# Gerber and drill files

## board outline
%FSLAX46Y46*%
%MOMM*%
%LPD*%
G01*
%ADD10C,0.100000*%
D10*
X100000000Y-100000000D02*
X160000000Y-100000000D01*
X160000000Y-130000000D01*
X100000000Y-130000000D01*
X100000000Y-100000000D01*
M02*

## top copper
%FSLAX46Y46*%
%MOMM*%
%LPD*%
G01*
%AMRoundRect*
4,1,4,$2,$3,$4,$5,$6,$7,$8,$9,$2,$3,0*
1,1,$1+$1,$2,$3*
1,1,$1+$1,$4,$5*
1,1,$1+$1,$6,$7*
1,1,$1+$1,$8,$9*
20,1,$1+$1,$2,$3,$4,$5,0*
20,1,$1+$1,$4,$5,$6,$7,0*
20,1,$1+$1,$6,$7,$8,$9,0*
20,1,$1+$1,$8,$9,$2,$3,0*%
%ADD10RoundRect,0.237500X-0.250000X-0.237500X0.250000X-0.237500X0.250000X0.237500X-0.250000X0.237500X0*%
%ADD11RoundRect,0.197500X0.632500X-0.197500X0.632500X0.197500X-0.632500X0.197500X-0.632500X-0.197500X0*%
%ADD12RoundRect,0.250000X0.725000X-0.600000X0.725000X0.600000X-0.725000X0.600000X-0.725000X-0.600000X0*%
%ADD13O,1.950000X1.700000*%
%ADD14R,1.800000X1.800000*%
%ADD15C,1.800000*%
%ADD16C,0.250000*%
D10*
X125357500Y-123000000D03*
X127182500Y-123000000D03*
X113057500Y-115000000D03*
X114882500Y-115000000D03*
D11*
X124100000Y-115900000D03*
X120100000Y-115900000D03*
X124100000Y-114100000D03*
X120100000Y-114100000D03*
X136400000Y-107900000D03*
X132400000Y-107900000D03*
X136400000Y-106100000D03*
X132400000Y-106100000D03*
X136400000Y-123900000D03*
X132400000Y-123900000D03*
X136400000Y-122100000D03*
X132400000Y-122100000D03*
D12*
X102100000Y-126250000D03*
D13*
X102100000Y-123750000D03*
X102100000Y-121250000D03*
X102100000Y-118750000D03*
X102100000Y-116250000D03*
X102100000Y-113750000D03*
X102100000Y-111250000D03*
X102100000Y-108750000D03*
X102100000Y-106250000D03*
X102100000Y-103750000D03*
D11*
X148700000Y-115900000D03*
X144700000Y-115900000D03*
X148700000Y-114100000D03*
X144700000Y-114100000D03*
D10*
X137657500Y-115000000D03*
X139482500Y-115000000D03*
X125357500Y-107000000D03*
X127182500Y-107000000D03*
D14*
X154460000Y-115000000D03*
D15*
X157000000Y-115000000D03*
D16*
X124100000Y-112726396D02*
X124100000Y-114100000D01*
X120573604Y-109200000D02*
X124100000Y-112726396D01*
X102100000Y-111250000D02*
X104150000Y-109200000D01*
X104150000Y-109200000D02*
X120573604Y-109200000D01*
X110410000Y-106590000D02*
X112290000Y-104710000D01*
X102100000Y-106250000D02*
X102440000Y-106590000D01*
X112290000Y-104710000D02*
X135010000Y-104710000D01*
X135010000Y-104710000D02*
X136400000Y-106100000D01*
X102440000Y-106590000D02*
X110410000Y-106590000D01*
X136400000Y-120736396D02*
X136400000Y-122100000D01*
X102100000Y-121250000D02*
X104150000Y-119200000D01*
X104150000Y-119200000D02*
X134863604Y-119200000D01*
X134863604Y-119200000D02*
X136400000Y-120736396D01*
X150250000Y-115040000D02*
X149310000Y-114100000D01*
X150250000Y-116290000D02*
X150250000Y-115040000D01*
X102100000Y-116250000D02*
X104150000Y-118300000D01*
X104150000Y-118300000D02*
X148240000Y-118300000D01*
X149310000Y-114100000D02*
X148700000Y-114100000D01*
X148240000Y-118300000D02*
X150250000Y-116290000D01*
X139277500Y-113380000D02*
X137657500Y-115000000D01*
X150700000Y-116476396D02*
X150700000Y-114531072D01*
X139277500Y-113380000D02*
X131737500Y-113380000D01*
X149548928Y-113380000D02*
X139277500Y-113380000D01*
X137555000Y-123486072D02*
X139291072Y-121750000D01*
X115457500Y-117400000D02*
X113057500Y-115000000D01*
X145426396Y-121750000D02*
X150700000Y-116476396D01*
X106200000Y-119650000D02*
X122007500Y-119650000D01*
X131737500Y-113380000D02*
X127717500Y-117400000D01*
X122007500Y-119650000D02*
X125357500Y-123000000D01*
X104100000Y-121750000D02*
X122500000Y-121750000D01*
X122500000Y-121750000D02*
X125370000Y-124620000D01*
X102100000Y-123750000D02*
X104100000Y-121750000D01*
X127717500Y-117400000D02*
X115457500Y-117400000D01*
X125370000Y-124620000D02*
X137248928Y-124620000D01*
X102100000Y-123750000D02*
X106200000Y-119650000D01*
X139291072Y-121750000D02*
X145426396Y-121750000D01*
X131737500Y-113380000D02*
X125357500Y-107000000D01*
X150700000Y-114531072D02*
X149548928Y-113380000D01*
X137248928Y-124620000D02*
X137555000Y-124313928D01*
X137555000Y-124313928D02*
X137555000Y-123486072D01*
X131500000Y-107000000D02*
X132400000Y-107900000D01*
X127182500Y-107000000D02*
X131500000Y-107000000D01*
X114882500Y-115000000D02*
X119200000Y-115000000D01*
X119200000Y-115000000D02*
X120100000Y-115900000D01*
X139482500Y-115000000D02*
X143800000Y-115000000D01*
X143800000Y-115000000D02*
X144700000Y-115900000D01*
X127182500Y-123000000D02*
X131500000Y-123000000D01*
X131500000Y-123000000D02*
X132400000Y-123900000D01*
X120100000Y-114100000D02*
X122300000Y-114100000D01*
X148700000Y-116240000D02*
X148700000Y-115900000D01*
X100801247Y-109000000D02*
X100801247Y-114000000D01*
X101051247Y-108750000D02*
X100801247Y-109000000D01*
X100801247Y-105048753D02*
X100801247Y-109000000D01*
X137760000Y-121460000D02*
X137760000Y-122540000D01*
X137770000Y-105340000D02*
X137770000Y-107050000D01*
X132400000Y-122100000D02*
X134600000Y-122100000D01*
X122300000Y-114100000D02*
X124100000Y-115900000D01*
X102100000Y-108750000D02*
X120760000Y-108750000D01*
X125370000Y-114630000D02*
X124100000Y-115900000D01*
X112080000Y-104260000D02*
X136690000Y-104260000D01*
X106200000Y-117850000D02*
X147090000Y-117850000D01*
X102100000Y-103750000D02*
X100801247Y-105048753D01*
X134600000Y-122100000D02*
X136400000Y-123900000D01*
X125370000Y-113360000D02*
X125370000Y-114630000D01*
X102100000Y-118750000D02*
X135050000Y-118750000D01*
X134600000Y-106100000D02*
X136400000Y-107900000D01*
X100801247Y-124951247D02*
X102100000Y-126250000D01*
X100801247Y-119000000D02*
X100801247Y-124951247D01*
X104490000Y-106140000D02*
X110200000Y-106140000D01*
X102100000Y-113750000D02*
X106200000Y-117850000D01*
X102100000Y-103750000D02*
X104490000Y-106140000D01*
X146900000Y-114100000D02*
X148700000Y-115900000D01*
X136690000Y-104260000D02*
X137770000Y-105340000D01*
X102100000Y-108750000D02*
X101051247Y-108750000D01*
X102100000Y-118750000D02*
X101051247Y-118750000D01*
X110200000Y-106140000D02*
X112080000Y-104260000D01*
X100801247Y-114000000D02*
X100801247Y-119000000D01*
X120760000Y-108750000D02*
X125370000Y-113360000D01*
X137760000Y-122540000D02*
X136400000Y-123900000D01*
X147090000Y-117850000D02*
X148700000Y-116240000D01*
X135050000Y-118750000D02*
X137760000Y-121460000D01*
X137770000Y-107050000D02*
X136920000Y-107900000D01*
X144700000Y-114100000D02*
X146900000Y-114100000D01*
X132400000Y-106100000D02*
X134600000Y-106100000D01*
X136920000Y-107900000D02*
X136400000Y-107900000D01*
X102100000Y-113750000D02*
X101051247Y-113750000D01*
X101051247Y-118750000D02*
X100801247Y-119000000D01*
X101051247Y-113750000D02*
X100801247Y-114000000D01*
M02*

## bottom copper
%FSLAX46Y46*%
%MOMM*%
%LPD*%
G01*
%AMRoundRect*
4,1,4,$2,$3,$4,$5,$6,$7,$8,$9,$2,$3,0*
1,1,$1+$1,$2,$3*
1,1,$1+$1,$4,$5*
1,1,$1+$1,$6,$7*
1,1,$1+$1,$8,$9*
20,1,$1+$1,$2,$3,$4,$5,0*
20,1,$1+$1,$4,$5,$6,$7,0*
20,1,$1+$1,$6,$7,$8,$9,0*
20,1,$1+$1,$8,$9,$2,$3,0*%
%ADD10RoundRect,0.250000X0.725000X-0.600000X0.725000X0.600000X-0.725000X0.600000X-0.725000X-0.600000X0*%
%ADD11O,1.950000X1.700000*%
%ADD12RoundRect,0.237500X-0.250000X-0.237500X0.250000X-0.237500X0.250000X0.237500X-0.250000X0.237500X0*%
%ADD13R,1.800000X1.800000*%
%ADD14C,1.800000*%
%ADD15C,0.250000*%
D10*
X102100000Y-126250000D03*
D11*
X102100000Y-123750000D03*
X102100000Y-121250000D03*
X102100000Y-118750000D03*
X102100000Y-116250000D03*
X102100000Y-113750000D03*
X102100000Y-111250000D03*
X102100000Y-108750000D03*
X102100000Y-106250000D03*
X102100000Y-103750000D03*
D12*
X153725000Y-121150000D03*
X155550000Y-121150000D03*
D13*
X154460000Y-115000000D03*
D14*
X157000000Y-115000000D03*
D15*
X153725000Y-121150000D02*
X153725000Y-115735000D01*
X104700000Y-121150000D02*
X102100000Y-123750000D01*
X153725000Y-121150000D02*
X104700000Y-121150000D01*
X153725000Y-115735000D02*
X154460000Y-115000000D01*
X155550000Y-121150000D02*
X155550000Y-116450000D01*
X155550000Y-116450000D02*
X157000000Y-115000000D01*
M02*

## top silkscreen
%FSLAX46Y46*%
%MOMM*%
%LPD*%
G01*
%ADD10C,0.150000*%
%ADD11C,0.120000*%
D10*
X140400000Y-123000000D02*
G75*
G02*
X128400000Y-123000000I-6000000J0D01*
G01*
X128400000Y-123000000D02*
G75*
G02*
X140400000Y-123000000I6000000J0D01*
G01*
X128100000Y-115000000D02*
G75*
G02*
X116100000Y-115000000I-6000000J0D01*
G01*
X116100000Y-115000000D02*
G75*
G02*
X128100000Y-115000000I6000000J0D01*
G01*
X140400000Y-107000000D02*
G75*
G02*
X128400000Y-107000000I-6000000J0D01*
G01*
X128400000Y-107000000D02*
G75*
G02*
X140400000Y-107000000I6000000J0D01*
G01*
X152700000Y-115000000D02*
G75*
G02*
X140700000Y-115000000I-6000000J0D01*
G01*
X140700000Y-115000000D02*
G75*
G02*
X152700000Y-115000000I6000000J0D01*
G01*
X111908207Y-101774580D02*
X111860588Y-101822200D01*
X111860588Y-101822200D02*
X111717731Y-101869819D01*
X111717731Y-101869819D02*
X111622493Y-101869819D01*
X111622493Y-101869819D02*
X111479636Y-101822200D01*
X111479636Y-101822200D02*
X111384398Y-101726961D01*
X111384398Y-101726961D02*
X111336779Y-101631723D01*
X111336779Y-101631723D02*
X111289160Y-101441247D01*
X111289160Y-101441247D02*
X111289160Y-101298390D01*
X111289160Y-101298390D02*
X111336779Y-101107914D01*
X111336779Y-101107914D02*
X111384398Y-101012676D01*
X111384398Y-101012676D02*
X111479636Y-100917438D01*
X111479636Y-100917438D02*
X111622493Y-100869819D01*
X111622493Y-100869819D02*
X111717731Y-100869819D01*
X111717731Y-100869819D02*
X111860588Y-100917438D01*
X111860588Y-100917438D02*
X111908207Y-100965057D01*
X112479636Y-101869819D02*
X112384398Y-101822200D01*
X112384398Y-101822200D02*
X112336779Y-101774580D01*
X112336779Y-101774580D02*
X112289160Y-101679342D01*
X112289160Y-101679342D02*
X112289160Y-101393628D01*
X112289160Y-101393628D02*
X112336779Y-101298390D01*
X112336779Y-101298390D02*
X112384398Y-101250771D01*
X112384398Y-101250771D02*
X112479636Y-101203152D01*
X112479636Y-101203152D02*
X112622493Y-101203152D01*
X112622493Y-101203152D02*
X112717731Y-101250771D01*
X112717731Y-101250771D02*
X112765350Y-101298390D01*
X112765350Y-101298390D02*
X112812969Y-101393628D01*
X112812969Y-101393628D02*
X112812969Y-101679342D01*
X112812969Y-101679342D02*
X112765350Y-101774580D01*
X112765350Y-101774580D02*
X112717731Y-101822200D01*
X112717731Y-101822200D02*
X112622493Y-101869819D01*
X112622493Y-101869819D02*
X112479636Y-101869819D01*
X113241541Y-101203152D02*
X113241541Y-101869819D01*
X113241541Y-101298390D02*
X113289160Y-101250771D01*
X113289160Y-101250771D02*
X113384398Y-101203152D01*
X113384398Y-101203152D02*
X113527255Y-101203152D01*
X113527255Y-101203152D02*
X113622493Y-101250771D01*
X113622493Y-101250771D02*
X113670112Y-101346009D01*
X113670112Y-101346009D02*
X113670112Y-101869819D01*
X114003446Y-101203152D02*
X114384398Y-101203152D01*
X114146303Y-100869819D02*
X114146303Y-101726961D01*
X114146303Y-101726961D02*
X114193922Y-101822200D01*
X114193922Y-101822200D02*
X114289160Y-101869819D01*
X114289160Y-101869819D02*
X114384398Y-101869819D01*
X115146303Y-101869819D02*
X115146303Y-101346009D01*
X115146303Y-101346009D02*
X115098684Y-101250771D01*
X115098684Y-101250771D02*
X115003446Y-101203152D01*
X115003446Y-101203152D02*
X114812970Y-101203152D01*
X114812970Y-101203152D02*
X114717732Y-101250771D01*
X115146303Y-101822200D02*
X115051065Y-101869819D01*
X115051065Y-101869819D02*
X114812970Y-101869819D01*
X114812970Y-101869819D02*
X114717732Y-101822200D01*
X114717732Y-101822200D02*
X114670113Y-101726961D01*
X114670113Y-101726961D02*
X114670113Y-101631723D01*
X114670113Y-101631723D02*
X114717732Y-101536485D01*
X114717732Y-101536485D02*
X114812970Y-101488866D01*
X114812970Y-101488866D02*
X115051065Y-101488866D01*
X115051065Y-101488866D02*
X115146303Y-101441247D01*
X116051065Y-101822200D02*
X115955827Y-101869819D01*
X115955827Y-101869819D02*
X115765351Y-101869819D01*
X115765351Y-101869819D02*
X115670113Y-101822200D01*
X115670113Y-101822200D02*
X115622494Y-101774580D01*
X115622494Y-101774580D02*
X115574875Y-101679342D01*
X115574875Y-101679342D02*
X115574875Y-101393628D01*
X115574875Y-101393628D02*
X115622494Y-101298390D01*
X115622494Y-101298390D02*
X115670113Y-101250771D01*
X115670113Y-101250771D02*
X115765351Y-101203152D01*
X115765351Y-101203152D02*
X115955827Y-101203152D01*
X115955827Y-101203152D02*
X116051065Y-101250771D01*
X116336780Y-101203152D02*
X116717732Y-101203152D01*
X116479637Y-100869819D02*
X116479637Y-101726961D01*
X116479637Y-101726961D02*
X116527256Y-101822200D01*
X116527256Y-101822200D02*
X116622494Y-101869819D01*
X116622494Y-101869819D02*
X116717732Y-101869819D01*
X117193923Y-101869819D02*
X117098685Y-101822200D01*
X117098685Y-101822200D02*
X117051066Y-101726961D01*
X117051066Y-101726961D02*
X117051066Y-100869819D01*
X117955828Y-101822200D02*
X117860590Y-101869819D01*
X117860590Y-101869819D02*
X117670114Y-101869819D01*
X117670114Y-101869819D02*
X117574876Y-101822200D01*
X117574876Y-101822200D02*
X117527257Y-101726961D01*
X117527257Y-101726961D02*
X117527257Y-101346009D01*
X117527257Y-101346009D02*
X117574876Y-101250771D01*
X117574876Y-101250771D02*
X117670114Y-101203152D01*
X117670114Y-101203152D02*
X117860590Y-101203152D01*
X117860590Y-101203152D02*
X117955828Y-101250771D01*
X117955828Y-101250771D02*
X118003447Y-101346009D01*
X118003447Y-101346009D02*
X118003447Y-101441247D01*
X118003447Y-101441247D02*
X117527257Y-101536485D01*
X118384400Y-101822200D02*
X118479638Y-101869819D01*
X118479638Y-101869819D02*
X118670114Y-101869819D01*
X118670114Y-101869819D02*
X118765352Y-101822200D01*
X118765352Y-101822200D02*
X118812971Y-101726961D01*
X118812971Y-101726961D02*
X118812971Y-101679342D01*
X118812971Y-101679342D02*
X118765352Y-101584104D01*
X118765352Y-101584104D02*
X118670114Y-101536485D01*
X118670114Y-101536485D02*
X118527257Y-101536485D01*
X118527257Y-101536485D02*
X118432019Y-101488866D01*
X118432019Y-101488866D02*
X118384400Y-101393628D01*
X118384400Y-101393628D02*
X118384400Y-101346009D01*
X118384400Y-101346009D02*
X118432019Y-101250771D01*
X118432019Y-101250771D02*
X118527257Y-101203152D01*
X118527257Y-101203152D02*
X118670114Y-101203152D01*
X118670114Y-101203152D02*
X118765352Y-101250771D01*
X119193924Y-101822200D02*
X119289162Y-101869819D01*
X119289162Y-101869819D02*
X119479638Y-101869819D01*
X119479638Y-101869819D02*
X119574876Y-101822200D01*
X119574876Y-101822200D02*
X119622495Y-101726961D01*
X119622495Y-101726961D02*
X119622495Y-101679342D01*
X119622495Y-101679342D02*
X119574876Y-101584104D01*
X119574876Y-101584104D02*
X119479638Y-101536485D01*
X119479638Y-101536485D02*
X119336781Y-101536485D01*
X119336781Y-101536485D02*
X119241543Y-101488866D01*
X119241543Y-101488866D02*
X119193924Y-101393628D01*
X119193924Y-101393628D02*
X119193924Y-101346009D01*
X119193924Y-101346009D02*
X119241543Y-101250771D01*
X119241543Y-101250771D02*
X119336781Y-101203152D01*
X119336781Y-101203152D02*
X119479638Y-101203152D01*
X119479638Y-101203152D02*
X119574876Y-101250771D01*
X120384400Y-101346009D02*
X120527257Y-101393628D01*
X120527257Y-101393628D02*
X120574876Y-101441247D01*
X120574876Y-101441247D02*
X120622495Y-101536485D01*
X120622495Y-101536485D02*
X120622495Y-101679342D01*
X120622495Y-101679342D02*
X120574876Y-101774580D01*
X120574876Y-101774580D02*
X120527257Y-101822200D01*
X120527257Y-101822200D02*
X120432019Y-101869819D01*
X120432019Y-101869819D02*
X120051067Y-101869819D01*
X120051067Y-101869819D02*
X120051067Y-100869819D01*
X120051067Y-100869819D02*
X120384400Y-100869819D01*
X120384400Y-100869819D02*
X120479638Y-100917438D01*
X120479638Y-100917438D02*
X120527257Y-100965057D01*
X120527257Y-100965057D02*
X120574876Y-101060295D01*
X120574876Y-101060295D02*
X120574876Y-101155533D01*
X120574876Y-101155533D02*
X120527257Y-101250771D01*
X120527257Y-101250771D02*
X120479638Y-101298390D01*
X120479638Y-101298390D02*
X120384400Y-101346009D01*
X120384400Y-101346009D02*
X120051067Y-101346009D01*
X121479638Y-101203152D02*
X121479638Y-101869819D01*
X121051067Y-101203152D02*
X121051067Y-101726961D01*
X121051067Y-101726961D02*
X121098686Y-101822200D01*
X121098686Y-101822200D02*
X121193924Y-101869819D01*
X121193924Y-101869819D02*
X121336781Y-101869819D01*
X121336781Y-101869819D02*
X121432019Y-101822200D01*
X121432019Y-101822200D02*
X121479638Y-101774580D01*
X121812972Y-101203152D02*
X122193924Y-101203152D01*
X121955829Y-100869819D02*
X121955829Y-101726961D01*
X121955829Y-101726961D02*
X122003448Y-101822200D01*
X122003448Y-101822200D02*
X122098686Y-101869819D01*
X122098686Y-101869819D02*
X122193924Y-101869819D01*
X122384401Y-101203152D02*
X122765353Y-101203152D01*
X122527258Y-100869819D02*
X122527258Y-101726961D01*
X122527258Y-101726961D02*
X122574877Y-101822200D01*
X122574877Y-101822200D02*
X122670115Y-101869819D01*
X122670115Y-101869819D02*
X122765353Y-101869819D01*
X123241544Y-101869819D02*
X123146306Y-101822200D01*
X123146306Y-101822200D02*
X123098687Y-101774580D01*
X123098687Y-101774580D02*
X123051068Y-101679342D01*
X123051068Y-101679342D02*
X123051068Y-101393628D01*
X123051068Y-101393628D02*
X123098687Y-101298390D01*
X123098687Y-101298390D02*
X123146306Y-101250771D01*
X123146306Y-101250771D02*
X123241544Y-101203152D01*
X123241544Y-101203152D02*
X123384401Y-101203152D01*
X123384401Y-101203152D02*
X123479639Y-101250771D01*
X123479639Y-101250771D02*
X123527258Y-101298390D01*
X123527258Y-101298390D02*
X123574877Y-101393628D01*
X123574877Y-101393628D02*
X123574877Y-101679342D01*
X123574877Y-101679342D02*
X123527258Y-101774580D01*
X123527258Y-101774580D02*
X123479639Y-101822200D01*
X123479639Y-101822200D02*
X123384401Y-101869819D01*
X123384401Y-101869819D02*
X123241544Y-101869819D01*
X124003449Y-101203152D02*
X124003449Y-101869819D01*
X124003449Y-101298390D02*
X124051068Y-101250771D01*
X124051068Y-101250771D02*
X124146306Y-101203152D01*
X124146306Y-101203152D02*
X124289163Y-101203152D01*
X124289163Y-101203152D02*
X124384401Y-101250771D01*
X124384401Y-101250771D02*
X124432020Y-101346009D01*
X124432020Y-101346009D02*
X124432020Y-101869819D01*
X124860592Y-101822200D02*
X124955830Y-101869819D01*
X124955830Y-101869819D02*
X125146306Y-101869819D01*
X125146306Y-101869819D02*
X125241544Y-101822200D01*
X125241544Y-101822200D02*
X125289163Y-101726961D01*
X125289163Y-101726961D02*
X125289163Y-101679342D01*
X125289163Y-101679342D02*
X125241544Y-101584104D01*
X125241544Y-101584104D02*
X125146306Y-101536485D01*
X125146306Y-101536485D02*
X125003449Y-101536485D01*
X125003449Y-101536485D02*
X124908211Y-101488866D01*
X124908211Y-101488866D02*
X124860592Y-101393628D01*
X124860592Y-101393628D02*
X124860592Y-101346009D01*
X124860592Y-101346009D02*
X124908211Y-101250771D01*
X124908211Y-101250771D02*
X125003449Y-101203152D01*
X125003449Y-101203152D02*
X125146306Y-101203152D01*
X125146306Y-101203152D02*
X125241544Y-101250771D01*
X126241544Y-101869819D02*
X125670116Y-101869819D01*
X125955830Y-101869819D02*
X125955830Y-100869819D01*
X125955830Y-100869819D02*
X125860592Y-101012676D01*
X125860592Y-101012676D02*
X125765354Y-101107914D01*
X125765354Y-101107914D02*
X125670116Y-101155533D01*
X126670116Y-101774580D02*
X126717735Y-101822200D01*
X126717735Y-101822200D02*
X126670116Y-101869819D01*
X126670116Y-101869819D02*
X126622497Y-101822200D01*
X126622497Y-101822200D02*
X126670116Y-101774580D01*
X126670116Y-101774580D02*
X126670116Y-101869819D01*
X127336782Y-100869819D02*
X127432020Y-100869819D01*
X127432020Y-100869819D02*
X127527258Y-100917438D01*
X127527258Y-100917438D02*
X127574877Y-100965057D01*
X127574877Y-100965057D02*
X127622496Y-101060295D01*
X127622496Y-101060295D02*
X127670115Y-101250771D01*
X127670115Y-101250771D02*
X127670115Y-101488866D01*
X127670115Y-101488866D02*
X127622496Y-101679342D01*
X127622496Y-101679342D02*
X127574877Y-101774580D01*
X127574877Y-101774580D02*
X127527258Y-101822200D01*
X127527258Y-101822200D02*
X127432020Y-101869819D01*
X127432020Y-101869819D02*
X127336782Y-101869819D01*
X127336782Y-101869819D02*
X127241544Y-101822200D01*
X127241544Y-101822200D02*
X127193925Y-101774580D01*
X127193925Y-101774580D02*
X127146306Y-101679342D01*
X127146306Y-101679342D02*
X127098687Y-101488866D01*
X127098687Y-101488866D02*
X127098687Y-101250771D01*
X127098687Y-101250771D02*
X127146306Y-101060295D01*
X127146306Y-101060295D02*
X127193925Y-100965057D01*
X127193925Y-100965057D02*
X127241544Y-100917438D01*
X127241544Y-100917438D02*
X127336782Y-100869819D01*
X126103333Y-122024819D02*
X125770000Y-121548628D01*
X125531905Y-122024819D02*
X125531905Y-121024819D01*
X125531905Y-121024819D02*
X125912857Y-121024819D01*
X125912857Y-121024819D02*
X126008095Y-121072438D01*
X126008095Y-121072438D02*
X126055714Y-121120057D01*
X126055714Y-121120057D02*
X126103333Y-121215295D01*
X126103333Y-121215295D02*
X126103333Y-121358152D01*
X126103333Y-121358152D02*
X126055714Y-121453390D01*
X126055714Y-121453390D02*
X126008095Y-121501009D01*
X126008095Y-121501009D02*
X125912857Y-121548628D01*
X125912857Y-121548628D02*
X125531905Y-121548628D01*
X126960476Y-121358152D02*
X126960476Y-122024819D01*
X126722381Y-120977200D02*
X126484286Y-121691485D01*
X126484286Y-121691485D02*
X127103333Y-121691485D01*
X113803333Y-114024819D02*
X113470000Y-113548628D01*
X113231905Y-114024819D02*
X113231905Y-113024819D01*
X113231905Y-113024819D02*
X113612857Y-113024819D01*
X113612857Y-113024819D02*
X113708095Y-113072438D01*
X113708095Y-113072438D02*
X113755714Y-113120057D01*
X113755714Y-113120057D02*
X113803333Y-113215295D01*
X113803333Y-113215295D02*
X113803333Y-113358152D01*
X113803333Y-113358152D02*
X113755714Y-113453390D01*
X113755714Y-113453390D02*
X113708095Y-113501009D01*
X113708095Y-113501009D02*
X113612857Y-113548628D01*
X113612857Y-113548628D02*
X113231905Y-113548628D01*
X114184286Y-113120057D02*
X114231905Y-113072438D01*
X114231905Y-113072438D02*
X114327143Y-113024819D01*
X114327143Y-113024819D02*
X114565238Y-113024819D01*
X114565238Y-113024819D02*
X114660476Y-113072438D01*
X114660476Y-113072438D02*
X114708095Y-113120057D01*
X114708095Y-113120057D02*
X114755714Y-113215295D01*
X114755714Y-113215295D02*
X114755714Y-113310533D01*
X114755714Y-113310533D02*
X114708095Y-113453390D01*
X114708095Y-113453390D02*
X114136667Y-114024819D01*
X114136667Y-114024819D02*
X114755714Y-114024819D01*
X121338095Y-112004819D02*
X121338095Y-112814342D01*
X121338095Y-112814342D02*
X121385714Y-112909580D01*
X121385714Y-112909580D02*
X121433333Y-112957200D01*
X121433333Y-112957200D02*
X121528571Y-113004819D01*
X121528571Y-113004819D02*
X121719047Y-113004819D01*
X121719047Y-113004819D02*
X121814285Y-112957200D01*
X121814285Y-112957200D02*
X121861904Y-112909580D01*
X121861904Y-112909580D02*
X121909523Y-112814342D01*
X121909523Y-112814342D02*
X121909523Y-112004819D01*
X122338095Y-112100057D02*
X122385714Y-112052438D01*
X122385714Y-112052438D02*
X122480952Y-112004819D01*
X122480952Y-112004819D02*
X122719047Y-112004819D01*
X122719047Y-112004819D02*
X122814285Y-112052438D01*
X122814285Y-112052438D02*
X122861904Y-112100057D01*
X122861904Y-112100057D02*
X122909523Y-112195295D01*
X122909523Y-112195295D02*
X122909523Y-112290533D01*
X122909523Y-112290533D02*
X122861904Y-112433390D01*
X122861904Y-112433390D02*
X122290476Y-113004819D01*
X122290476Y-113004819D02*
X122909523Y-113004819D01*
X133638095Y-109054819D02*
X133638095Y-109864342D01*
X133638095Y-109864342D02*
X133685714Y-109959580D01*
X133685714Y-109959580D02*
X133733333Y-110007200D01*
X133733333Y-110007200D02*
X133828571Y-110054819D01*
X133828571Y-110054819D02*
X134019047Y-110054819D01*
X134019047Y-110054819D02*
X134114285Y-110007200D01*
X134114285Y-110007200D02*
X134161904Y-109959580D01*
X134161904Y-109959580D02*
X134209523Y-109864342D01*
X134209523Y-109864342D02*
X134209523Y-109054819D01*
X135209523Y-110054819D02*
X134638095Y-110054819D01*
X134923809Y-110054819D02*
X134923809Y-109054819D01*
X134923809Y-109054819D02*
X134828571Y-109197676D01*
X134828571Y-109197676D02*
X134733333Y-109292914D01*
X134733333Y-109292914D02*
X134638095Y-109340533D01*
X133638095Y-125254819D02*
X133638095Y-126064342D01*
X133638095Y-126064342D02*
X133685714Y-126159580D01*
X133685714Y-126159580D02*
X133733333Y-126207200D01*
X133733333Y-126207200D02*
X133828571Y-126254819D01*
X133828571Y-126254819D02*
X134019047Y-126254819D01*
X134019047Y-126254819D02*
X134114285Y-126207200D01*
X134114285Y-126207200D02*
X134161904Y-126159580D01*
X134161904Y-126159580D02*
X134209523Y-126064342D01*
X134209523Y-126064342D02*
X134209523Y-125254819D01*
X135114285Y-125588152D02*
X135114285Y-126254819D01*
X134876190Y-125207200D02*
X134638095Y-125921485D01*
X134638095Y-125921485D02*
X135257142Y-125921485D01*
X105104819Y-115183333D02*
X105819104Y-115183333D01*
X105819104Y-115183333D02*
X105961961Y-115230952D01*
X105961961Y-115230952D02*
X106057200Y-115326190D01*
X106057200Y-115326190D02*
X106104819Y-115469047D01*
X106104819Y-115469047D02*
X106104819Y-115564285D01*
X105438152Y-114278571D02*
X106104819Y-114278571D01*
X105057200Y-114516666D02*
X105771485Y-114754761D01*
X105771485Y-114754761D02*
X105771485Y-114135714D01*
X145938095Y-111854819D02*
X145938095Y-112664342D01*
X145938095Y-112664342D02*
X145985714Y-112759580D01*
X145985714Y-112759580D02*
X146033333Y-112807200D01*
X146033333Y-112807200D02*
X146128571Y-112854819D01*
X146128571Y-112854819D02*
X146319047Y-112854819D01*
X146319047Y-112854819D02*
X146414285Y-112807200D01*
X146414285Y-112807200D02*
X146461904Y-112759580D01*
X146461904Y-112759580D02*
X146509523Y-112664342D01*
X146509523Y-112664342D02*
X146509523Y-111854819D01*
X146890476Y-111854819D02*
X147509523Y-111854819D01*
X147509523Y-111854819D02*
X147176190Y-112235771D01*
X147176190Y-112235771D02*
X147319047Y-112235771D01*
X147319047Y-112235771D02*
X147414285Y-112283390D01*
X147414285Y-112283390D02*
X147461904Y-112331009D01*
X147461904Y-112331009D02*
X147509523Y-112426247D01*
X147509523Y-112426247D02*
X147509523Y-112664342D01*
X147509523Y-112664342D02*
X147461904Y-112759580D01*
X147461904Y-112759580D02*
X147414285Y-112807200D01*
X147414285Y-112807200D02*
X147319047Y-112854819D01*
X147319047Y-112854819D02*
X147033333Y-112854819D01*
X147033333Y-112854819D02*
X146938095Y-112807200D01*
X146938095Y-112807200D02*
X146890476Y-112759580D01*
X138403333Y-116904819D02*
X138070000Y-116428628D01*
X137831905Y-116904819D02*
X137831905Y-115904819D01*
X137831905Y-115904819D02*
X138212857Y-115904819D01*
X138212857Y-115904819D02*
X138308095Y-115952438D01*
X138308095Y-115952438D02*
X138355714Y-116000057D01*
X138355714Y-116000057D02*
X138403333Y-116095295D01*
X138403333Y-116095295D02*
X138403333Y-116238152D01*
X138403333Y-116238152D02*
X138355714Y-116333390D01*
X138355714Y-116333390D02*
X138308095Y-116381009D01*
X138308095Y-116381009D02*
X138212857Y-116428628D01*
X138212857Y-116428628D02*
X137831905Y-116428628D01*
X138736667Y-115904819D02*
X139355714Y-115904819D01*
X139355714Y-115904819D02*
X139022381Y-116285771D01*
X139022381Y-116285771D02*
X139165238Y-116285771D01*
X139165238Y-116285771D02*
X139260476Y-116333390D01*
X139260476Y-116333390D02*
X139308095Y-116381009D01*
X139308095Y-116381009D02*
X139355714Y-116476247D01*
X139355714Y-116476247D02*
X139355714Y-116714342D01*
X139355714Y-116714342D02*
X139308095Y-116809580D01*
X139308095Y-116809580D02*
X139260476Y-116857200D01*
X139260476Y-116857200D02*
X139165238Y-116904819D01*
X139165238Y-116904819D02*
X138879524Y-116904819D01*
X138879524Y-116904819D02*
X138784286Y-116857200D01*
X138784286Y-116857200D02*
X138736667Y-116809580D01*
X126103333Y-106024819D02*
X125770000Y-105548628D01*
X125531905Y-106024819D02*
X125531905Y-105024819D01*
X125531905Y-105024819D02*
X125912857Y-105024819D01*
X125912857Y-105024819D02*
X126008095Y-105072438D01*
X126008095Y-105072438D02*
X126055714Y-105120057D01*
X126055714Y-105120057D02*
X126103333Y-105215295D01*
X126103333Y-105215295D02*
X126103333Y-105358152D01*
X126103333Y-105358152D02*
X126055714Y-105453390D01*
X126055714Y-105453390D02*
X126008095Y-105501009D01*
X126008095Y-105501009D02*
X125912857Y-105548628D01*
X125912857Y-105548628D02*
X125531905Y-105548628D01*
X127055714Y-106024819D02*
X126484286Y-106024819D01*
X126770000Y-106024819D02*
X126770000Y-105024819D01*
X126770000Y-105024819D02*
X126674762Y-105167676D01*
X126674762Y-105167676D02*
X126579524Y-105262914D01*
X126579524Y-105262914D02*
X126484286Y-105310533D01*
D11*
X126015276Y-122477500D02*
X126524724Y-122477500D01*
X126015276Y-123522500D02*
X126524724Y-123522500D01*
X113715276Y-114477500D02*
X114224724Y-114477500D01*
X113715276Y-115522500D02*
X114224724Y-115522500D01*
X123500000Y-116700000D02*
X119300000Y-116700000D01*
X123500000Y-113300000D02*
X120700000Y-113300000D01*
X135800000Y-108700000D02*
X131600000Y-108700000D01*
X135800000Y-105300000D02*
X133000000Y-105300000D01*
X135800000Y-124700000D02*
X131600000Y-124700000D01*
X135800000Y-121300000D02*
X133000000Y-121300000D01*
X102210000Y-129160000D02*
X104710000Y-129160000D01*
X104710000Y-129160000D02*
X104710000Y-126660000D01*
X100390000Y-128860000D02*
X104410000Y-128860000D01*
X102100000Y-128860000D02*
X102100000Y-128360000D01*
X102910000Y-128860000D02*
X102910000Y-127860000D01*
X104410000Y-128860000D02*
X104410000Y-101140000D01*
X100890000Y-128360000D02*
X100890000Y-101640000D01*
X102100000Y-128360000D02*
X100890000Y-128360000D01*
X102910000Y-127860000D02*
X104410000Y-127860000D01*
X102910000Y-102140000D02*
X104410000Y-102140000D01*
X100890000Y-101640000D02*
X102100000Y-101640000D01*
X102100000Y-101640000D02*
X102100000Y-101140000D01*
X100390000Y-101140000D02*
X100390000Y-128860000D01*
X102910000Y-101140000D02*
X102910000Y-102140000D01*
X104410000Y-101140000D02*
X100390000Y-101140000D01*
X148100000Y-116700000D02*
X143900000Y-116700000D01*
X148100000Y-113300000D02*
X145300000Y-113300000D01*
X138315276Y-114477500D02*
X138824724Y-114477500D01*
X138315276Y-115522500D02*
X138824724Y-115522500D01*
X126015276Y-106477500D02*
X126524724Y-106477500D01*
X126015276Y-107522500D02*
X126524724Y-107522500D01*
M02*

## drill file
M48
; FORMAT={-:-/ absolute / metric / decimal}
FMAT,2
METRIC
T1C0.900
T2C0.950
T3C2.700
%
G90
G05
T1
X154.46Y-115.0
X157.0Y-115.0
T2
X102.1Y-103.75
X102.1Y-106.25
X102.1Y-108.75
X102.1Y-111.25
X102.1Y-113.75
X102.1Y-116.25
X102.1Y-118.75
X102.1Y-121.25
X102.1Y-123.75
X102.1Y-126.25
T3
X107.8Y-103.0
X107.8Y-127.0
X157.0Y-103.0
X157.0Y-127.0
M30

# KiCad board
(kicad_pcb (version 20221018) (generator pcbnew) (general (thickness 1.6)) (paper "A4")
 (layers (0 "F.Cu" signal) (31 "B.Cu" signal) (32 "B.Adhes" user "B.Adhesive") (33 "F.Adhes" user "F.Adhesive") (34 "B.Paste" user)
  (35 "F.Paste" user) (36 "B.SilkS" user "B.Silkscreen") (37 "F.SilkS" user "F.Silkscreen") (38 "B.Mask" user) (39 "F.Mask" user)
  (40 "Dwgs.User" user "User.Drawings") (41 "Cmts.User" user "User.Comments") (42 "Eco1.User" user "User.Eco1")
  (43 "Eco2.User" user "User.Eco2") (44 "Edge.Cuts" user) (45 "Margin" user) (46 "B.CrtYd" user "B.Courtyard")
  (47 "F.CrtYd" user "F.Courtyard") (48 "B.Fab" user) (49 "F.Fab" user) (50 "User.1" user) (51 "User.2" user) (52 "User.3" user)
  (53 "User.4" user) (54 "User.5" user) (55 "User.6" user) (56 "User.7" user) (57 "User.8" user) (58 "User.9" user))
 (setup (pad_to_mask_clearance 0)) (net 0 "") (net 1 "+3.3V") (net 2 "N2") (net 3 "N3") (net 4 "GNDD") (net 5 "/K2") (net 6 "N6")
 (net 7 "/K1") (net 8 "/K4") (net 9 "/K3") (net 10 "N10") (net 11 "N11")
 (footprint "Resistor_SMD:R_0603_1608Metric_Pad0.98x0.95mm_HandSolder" (layer "F.Cu") (at 126.27 123)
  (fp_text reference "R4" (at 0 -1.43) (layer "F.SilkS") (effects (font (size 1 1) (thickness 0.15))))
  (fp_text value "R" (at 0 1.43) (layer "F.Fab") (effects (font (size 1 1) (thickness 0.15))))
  (fp_line (start -0.254724 -0.5225) (end 0.254724 -0.5225) (stroke (width 0.12) (type solid)) (layer "F.SilkS"))
  (fp_line (start -0.254724 0.5225) (end 0.254724 0.5225) (stroke (width 0.12) (type solid)) (layer "F.SilkS"))
  (pad "1" smd roundrect (at -0.9125 0) (size 0.975 0.95) (layers "F.Cu" "F.Paste" "F.Mask") (roundrect_rratio 0.25) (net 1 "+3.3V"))
  (pad "2" smd roundrect (at 0.9125 0) (size 0.975 0.95) (layers "F.Cu" "F.Paste" "F.Mask") (roundrect_rratio 0.25) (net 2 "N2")))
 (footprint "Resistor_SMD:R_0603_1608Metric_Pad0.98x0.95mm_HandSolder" (layer "F.Cu") (at 113.97 115)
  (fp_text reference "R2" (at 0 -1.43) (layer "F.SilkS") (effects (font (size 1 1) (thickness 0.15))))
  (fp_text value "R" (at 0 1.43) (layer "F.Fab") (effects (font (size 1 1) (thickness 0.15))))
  (fp_line (start -0.254724 -0.5225) (end 0.254724 -0.5225) (stroke (width 0.12) (type solid)) (layer "F.SilkS"))
  (fp_line (start -0.254724 0.5225) (end 0.254724 0.5225) (stroke (width 0.12) (type solid)) (layer "F.SilkS"))
  (pad "1" smd roundrect (at -0.9125 0) (size 0.975 0.95) (layers "F.Cu" "F.Paste" "F.Mask") (roundrect_rratio 0.25) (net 1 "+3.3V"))
  (pad "2" smd roundrect (at 0.9125 0) (size 0.975 0.95) (layers "F.Cu" "F.Paste" "F.Mask") (roundrect_rratio 0.25) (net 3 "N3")))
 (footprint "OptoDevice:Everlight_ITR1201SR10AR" (layer "F.Cu") (at 122.1 115 90)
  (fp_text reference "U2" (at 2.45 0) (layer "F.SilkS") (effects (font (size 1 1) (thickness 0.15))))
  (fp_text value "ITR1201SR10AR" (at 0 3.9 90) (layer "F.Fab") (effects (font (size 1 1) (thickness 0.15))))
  (fp_line (start -1.7 1.4) (end -1.7 -2.8) (stroke (width 0.12) (type solid)) (layer "F.SilkS"))
  (fp_line (start 1.7 1.4) (end 1.7 -1.4) (stroke (width 0.12) (type solid)) (layer "F.SilkS"))
  (pad "1" smd roundrect (at -0.9 2 90) (size 0.79 1.66) (layers "F.Cu" "F.Paste" "F.Mask") (roundrect_rratio 0.25) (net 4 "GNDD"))
  (pad "2" smd roundrect (at -0.9 -2 90) (size 0.79 1.66) (layers "F.Cu" "F.Paste" "F.Mask") (roundrect_rratio 0.25) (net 3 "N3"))
  (pad "3" smd roundrect (at 0.9 2 90) (size 0.79 1.66) (layers "F.Cu" "F.Paste" "F.Mask") (roundrect_rratio 0.25) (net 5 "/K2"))
  (pad "4" smd roundrect (at 0.9 -2 90) (size 0.79 1.66) (layers "F.Cu" "F.Paste" "F.Mask") (roundrect_rratio 0.25) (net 4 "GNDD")))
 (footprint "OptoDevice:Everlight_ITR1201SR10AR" (layer "F.Cu") (at 134.4 107 90)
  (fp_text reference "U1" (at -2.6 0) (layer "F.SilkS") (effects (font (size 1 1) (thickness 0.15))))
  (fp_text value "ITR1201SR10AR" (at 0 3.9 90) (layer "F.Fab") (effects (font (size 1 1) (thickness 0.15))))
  (fp_line (start -1.7 1.4) (end -1.7 -2.8) (stroke (width 0.12) (type solid)) (layer "F.SilkS"))
  (fp_line (start 1.7 1.4) (end 1.7 -1.4) (stroke (width 0.12) (type solid)) (layer "F.SilkS"))
  (pad "1" smd roundrect (at -0.9 2 90) (size 0.79 1.66) (layers "F.Cu" "F.Paste" "F.Mask") (roundrect_rratio 0.25) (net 4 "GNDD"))
  (pad "2" smd roundrect (at -0.9 -2 90) (size 0.79 1.66) (layers "F.Cu" "F.Paste" "F.Mask") (roundrect_rratio 0.25) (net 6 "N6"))
  (pad "3" smd roundrect (at 0.9 2 90) (size 0.79 1.66) (layers "F.Cu" "F.Paste" "F.Mask") (roundrect_rratio 0.25) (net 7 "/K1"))
  (pad "4" smd roundrect (at 0.9 -2 90) (size 0.79 1.66) (layers "F.Cu" "F.Paste" "F.Mask") (roundrect_rratio 0.25) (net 4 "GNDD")))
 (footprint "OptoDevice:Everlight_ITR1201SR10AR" (layer "F.Cu") (at 134.4 123 90)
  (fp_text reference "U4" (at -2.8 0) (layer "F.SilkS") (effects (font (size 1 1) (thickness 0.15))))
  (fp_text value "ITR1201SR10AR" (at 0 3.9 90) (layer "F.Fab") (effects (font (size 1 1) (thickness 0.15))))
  (fp_line (start -1.7 1.4) (end -1.7 -2.8) (stroke (width 0.12) (type solid)) (layer "F.SilkS"))
  (fp_line (start 1.7 1.4) (end 1.7 -1.4) (stroke (width 0.12) (type solid)) (layer "F.SilkS"))
  (pad "1" smd roundrect (at -0.9 2 90) (size 0.79 1.66) (layers "F.Cu" "F.Paste" "F.Mask") (roundrect_rratio 0.25) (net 4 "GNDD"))
  (pad "2" smd roundrect (at -0.9 -2 90) (size 0.79 1.66) (layers "F.Cu" "F.Paste" "F.Mask") (roundrect_rratio 0.25) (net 2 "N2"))
  (pad "3" smd roundrect (at 0.9 2 90) (size 0.79 1.66) (layers "F.Cu" "F.Paste" "F.Mask") (roundrect_rratio 0.25) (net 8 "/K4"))
  (pad "4" smd roundrect (at 0.9 -2 90) (size 0.79 1.66) (layers "F.Cu" "F.Paste" "F.Mask") (roundrect_rratio 0.25) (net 4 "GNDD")))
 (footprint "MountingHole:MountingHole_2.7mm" (layer "F.Cu") (at 107.8 103)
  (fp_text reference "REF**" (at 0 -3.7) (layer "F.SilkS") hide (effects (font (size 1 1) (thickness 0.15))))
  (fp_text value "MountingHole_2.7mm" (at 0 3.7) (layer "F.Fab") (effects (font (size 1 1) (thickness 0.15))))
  (pad "" np_thru_hole circle (at 0 0) (size 2.7 2.7) (drill 2.7) (layers "F&B.Cu" "*.Mask")))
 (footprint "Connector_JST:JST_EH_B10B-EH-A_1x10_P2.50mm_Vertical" (layer "F.Cu") (at 102.1 126.25 90)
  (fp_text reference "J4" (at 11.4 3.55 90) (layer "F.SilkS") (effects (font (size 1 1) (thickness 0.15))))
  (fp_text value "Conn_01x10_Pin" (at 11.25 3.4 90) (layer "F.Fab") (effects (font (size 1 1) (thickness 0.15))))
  (fp_line (start -2.91 0.11) (end -2.91 2.61) (stroke (width 0.12) (type solid)) (layer "F.SilkS"))
  (fp_line (start -2.91 2.61) (end -0.41 2.61) (stroke (width 0.12) (type solid)) (layer "F.SilkS"))
  (fp_line (start -2.61 -1.71) (end -2.61 2.31) (stroke (width 0.12) (type solid)) (layer "F.SilkS"))
  (fp_line (start -2.61 0) (end -2.11 0) (stroke (width 0.12) (type solid)) (layer "F.SilkS"))
  (fp_line (start -2.61 0.81) (end -1.61 0.81) (stroke (width 0.12) (type solid)) (layer "F.SilkS"))
  (fp_line (start -2.61 2.31) (end 25.11 2.31) (stroke (width 0.12) (type solid)) (layer "F.SilkS"))
  (fp_line (start -2.11 -1.21) (end 24.61 -1.21) (stroke (width 0.12) (type solid)) (layer "F.SilkS"))
  (fp_line (start -2.11 0) (end -2.11 -1.21) (stroke (width 0.12) (type solid)) (layer "F.SilkS"))
  (fp_line (start -1.61 0.81) (end -1.61 2.31) (stroke (width 0.12) (type solid)) (layer "F.SilkS"))
  (fp_line (start 24.11 0.81) (end 24.11 2.31) (stroke (width 0.12) (type solid)) (layer "F.SilkS"))
  (fp_line (start 24.61 -1.21) (end 24.61 0) (stroke (width 0.12) (type solid)) (layer "F.SilkS"))
  (fp_line (start 24.61 0) (end 25.11 0) (stroke (width 0.12) (type solid)) (layer "F.SilkS"))
  (fp_line (start 25.11 -1.71) (end -2.61 -1.71) (stroke (width 0.12) (type solid)) (layer "F.SilkS"))
  (fp_line (start 25.11 0.81) (end 24.11 0.81) (stroke (width 0.12) (type solid)) (layer "F.SilkS"))
  (fp_line (start 25.11 2.31) (end 25.11 -1.71) (stroke (width 0.12) (type solid)) (layer "F.SilkS"))
  (pad "1" thru_hole roundrect (at 0 0 90) (size 1.7 1.95) (drill 0.95) (layers "*.Cu" "*.Mask") (roundrect_rratio 0.147059) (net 4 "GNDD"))
  (pad "2" thru_hole oval (at 2.5 0 90) (size 1.7 1.95) (drill 0.95) (layers "*.Cu" "*.Mask") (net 1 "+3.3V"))
  (pad "3" thru_hole oval (at 5 0 90) (size 1.7 1.95) (drill 0.95) (layers "*.Cu" "*.Mask") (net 8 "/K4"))
  (pad "4" thru_hole oval (at 7.5 0 90) (size 1.7 1.95) (drill 0.95) (layers "*.Cu" "*.Mask") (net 4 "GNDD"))
  (pad "5" thru_hole oval (at 10 0 90) (size 1.7 1.95) (drill 0.95) (layers "*.Cu" "*.Mask") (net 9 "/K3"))
  (pad "6" thru_hole oval (at 12.5 0 90) (size 1.7 1.95) (drill 0.95) (layers "*.Cu" "*.Mask") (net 4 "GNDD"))
  (pad "7" thru_hole oval (at 15 0 90) (size 1.7 1.95) (drill 0.95) (layers "*.Cu" "*.Mask") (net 5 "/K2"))
  (pad "8" thru_hole oval (at 17.5 0 90) (size 1.7 1.95) (drill 0.95) (layers "*.Cu" "*.Mask") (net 4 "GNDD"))
  (pad "9" thru_hole oval (at 20 0 90) (size 1.7 1.95) (drill 0.95) (layers "*.Cu" "*.Mask") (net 7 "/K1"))
  (pad "10" thru_hole oval (at 22.5 0 90) (size 1.7 1.95) (drill 0.95) (layers "*.Cu" "*.Mask") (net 4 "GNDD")))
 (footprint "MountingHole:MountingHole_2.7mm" (layer "F.Cu") (at 157 103)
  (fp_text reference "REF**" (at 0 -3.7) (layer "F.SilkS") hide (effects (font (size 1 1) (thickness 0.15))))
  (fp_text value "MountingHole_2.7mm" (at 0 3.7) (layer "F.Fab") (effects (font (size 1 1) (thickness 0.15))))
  (pad "" np_thru_hole circle (at 0 0) (size 2.7 2.7) (drill 2.7) (layers "*.Cu" "*.Mask")))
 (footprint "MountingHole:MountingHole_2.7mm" (layer "F.Cu") (at 107.8 127)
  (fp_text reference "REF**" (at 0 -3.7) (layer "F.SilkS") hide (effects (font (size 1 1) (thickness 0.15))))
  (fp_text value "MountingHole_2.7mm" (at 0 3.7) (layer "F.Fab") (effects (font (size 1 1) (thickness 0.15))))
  (pad "" np_thru_hole circle (at 0 0) (size 2.7 2.7) (drill 2.7) (layers "F&B.Cu" "*.Mask")))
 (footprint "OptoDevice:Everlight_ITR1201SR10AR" (layer "F.Cu") (at 146.7 115 90)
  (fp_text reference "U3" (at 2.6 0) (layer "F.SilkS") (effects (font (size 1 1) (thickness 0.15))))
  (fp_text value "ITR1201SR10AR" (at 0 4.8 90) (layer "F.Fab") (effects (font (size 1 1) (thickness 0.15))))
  (fp_line (start -1.7 1.4) (end -1.7 -2.8) (stroke (width 0.12) (type solid)) (layer "F.SilkS"))
  (fp_line (start 1.7 1.4) (end 1.7 -1.4) (stroke (width 0.12) (type solid)) (layer "F.SilkS"))
  (pad "1" smd roundrect (at -0.9 2 90) (size 0.79 1.66) (layers "F.Cu" "F.Paste" "F.Mask") (roundrect_rratio 0.25) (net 4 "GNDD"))
  (pad "2" smd roundrect (at -0.9 -2 90) (size 0.79 1.66) (layers "F.Cu" "F.Paste" "F.Mask") (roundrect_rratio 0.25) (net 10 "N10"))
  (pad "3" smd roundrect (at 0.9 2 90) (size 0.79 1.66) (layers "F.Cu" "F.Paste" "F.Mask") (roundrect_rratio 0.25) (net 9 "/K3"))
  (pad "4" smd roundrect (at 0.9 -2 90) (size 0.79 1.66) (layers "F.Cu" "F.Paste" "F.Mask") (roundrect_rratio 0.25) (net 4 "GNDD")))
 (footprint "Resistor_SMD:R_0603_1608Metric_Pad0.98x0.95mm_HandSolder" (layer "F.Cu") (at 138.57 115)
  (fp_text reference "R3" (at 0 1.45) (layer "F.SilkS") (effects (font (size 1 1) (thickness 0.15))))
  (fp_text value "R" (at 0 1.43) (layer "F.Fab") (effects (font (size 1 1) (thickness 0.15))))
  (fp_line (start -0.254724 -0.5225) (end 0.254724 -0.5225) (stroke (width 0.12) (type solid)) (layer "F.SilkS"))
  (fp_line (start -0.254724 0.5225) (end 0.254724 0.5225) (stroke (width 0.12) (type solid)) (layer "F.SilkS"))
  (pad "1" smd roundrect (at -0.9125 0) (size 0.975 0.95) (layers "F.Cu" "F.Paste" "F.Mask") (roundrect_rratio 0.25) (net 1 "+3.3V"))
  (pad "2" smd roundrect (at 0.9125 0) (size 0.975 0.95) (layers "F.Cu" "F.Paste" "F.Mask") (roundrect_rratio 0.25) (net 10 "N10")))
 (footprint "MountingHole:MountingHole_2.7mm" (layer "F.Cu") (at 157 127)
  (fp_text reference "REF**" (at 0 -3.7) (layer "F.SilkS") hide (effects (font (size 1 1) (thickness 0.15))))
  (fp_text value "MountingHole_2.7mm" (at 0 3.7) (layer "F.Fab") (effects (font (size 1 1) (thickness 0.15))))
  (pad "" np_thru_hole circle (at 0 0) (size 2.7 2.7) (drill 2.7) (layers "F&B.Cu" "*.Mask")))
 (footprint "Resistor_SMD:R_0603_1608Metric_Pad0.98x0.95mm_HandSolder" (layer "F.Cu") (at 126.27 107)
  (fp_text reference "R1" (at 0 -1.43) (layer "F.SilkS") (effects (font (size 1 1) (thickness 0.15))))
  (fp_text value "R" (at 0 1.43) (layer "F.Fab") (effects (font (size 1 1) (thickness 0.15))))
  (fp_line (start -0.254724 -0.5225) (end 0.254724 -0.5225) (stroke (width 0.12) (type solid)) (layer "F.SilkS"))
  (fp_line (start -0.254724 0.5225) (end 0.254724 0.5225) (stroke (width 0.12) (type solid)) (layer "F.SilkS"))
  (pad "1" smd roundrect (at -0.9125 0) (size 0.975 0.95) (layers "F.Cu" "F.Paste" "F.Mask") (roundrect_rratio 0.25) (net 1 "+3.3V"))
  (pad "2" smd roundrect (at 0.9125 0) (size 0.975 0.95) (layers "F.Cu" "F.Paste" "F.Mask") (roundrect_rratio 0.25) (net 6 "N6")))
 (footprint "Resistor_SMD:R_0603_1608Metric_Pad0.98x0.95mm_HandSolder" (layer "B.Cu") (at 154.6375 121.15)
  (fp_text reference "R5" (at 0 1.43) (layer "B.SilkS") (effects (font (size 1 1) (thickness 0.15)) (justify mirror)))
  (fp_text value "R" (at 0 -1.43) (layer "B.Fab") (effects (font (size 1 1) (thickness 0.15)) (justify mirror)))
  (pad "1" smd roundrect (at -0.9125 0) (size 0.975 0.95) (layers "B.Cu" "B.Paste" "B.Mask") (roundrect_rratio 0.25) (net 1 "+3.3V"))
  (pad "2" smd roundrect (at 0.9125 0) (size 0.975 0.95) (layers "B.Cu" "B.Paste" "B.Mask") (roundrect_rratio 0.25) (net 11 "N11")))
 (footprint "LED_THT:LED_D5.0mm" (layer "B.Cu") (at 154.46 115)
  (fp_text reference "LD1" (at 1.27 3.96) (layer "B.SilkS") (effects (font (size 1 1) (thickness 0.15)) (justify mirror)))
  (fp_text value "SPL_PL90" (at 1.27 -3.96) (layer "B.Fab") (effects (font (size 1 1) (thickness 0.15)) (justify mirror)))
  (pad "1" thru_hole rect (at 0 0) (size 1.8 1.8) (drill 0.9) (layers "*.Cu" "F.Mask") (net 1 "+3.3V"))
  (pad "2" thru_hole circle (at 2.54 0) (size 1.8 1.8) (drill 0.9) (layers "*.Cu" "F.Mask") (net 11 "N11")))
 (gr_circle (center 134.4 123) (end 134.4 117) (stroke (width 0.15) (type default)) (fill none) (layer "F.SilkS"))
 (gr_circle (center 122.1 115) (end 122.1 109) (stroke (width 0.15) (type default)) (fill none) (layer "F.SilkS"))
 (gr_circle (center 134.4 107) (end 134.4 113) (stroke (width 0.15) (type default)) (fill none) (layer "F.SilkS"))
 (gr_circle (center 146.7 115) (end 146.7 109) (stroke (width 0.15) (type default)) (fill none) (layer "F.SilkS"))
 (gr_rect (start 100 100) (end 160 130) (stroke (width 0.1) (type default)) (fill none) (layer "Edge.Cuts"))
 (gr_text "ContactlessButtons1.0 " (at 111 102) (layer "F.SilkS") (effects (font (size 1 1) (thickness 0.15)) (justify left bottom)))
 (segment (start 124.1 112.726396) (end 124.1 114.1) (width 0.25) (layer "F.Cu") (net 5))
 (segment (start 120.573604 109.2) (end 124.1 112.726396) (width 0.25) (layer "F.Cu") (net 5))
 (segment (start 102.1 111.25) (end 104.15 109.2) (width 0.25) (layer "F.Cu") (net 5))
 (segment (start 104.15 109.2) (end 120.573604 109.2) (width 0.25) (layer "F.Cu") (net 5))
 (segment (start 110.41 106.59) (end 112.29 104.71) (width 0.25) (layer "F.Cu") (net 7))
 (segment (start 102.1 106.25) (end 102.44 106.59) (width 0.25) (layer "F.Cu") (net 7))
 (segment (start 112.29 104.71) (end 135.01 104.71) (width 0.25) (layer "F.Cu") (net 7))
 (segment (start 135.01 104.71) (end 136.4 106.1) (width 0.25) (layer "F.Cu") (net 7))
 (segment (start 102.44 106.59) (end 110.41 106.59) (width 0.25) (layer "F.Cu") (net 7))
 (segment (start 136.4 120.736396) (end 136.4 122.1) (width 0.25) (layer "F.Cu") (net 8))
 (segment (start 102.1 121.25) (end 104.15 119.2) (width 0.25) (layer "F.Cu") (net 8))
 (segment (start 104.15 119.2) (end 134.863604 119.2) (width 0.25) (layer "F.Cu") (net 8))
 (segment (start 134.863604 119.2) (end 136.4 120.736396) (width 0.25) (layer "F.Cu") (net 8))
 (segment (start 150.25 115.04) (end 149.31 114.1) (width 0.25) (layer "F.Cu") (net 9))
 (segment (start 150.25 116.29) (end 150.25 115.04) (width 0.25) (layer "F.Cu") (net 9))
 (segment (start 102.1 116.25) (end 104.15 118.3) (width 0.25) (layer "F.Cu") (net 9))
 (segment (start 104.15 118.3) (end 148.24 118.3) (width 0.25) (layer "F.Cu") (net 9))
 (segment (start 149.31 114.1) (end 148.7 114.1) (width 0.25) (layer "F.Cu") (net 9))
 (segment (start 148.24 118.3) (end 150.25 116.29) (width 0.25) (layer "F.Cu") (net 9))
 (segment (start 139.2775 113.38) (end 137.6575 115) (width 0.25) (layer "F.Cu") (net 1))
 (segment (start 150.7 116.476396) (end 150.7 114.531072) (width 0.25) (layer "F.Cu") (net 1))
 (segment (start 139.2775 113.38) (end 131.7375 113.38) (width 0.25) (layer "F.Cu") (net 1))
 (segment (start 149.548928 113.38) (end 139.2775 113.38) (width 0.25) (layer "F.Cu") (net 1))
 (segment (start 137.555 123.486072) (end 139.291072 121.75) (width 0.25) (layer "F.Cu") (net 1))
 (segment (start 115.4575 117.4) (end 113.0575 115) (width 0.25) (layer "F.Cu") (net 1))
 (segment (start 145.426396 121.75) (end 150.7 116.476396) (width 0.25) (layer "F.Cu") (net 1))
 (segment (start 106.2 119.65) (end 122.0075 119.65) (width 0.25) (layer "F.Cu") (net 1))
 (segment (start 131.7375 113.38) (end 127.7175 117.4) (width 0.25) (layer "F.Cu") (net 1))
 (segment (start 122.0075 119.65) (end 125.3575 123) (width 0.25) (layer "F.Cu") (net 1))
 (segment (start 104.1 121.75) (end 122.5 121.75) (width 0.25) (layer "F.Cu") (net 1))
 (segment (start 122.5 121.75) (end 125.37 124.62) (width 0.25) (layer "F.Cu") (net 1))
 (segment (start 102.1 123.75) (end 104.1 121.75) (width 0.25) (layer "F.Cu") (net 1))
 (segment (start 127.7175 117.4) (end 115.4575 117.4) (width 0.25) (layer "F.Cu") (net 1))
 (segment (start 125.37 124.62) (end 137.248928 124.62) (width 0.25) (layer "F.Cu") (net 1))
 (segment (start 102.1 123.75) (end 106.2 119.65) (width 0.25) (layer "F.Cu") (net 1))
 (segment (start 139.291072 121.75) (end 145.426396 121.75) (width 0.25) (layer "F.Cu") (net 1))
 (segment (start 131.7375 113.38) (end 125.3575 107) (width 0.25) (layer "F.Cu") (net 1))
 (segment (start 150.7 114.531072) (end 149.548928 113.38) (width 0.25) (layer "F.Cu") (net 1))
 (segment (start 137.248928 124.62) (end 137.555 124.313928) (width 0.25) (layer "F.Cu") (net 1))
 (segment (start 137.555 124.313928) (end 137.555 123.486072) (width 0.25) (layer "F.Cu") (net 1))
 (segment (start 153.725 121.15) (end 153.725 115.735) (width 0.25) (layer "B.Cu") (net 1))
 (segment (start 104.7 121.15) (end 102.1 123.75) (width 0.25) (layer "B.Cu") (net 1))
 (segment (start 153.725 121.15) (end 104.7 121.15) (width 0.25) (layer "B.Cu") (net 1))
 (segment (start 153.725 115.735) (end 154.46 115) (width 0.25) (layer "B.Cu") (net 1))
 (segment (start 131.5 107) (end 132.4 107.9) (width 0.25) (layer "F.Cu") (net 6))
 (segment (start 127.1825 107) (end 131.5 107) (width 0.25) (layer "F.Cu") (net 6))
 (segment (start 114.8825 115) (end 119.2 115) (width 0.25) (layer "F.Cu") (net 3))
 (segment (start 119.2 115) (end 120.1 115.9) (width 0.25) (layer "F.Cu") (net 3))
 (segment (start 139.4825 115) (end 143.8 115) (width 0.25) (layer "F.Cu") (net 10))
 (segment (start 143.8 115) (end 144.7 115.9) (width 0.25) (layer "F.Cu") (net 10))
 (segment (start 127.1825 123) (end 131.5 123) (width 0.25) (layer "F.Cu") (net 2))
 (segment (start 131.5 123) (end 132.4 123.9) (width 0.25) (layer "F.Cu") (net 2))
 (segment (start 120.1 114.1) (end 122.3 114.1) (width 0.25) (layer "F.Cu") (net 4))
 (segment (start 148.7 116.24) (end 148.7 115.9) (width 0.25) (layer "F.Cu") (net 4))
 (segment (start 100.801247 109) (end 100.801247 114) (width 0.25) (layer "F.Cu") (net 4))
 (segment (start 101.051247 108.75) (end 100.801247 109) (width 0.25) (layer "F.Cu") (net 4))
 (segment (start 100.801247 105.048753) (end 100.801247 109) (width 0.25) (layer "F.Cu") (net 4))
 (segment (start 137.76 121.46) (end 137.76 122.54) (width 0.25) (layer "F.Cu") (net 4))
 (segment (start 137.77 105.34) (end 137.77 107.05) (width 0.25) (layer "F.Cu") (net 4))
 (segment (start 132.4 122.1) (end 134.6 122.1) (width 0.25) (layer "F.Cu") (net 4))
 (segment (start 122.3 114.1) (end 124.1 115.9) (width 0.25) (layer "F.Cu") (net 4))
 (segment (start 102.1 108.75) (end 120.76 108.75) (width 0.25) (layer "F.Cu") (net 4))
 (segment (start 125.37 114.63) (end 124.1 115.9) (width 0.25) (layer "F.Cu") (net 4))
 (segment (start 112.08 104.26) (end 136.69 104.26) (width 0.25) (layer "F.Cu") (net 4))
 (segment (start 106.2 117.85) (end 147.09 117.85) (width 0.25) (layer "F.Cu") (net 4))
 (segment (start 102.1 103.75) (end 100.801247 105.048753) (width 0.25) (layer "F.Cu") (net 4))
 (segment (start 134.6 122.1) (end 136.4 123.9) (width 0.25) (layer "F.Cu") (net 4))
 (segment (start 125.37 113.36) (end 125.37 114.63) (width 0.25) (layer "F.Cu") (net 4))
 (segment (start 102.1 118.75) (end 135.05 118.75) (width 0.25) (layer "F.Cu") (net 4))
 (segment (start 134.6 106.1) (end 136.4 107.9) (width 0.25) (layer "F.Cu") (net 4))
 (segment (start 100.801247 124.951247) (end 102.1 126.25) (width 0.25) (layer "F.Cu") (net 4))
 (segment (start 100.801247 119) (end 100.801247 124.951247) (width 0.25) (layer "F.Cu") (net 4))
 (segment (start 104.49 106.14) (end 110.2 106.14) (width 0.25) (layer "F.Cu") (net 4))
 (segment (start 102.1 113.75) (end 106.2 117.85) (width 0.25) (layer "F.Cu") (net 4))
 (segment (start 102.1 103.75) (end 104.49 106.14) (width 0.25) (layer "F.Cu") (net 4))
 (segment (start 146.9 114.1) (end 148.7 115.9) (width 0.25) (layer "F.Cu") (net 4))
 (segment (start 136.69 104.26) (end 137.77 105.34) (width 0.25) (layer "F.Cu") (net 4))
 (segment (start 102.1 108.75) (end 101.051247 108.75) (width 0.25) (layer "F.Cu") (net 4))
 (segment (start 102.1 118.75) (end 101.051247 118.75) (width 0.25) (layer "F.Cu") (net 4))
 (segment (start 110.2 106.14) (end 112.08 104.26) (width 0.25) (layer "F.Cu") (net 4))
 (segment (start 100.801247 114) (end 100.801247 119) (width 0.25) (layer "F.Cu") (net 4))
 (segment (start 120.76 108.75) (end 125.37 113.36) (width 0.25) (layer "F.Cu") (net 4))
 (segment (start 137.76 122.54) (end 136.4 123.9) (width 0.25) (layer "F.Cu") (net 4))
 (segment (start 147.09 117.85) (end 148.7 116.24) (width 0.25) (layer "F.Cu") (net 4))
 (segment (start 135.05 118.75) (end 137.76 121.46) (width 0.25) (layer "F.Cu") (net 4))
 (segment (start 137.77 107.05) (end 136.92 107.9) (width 0.25) (layer "F.Cu") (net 4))
 (segment (start 144.7 114.1) (end 146.9 114.1) (width 0.25) (layer "F.Cu") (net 4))
 (segment (start 132.4 106.1) (end 134.6 106.1) (width 0.25) (layer "F.Cu") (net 4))
 (segment (start 136.92 107.9) (end 136.4 107.9) (width 0.25) (layer "F.Cu") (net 4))
 (segment (start 102.1 113.75) (end 101.051247 113.75) (width 0.25) (layer "F.Cu") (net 4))
 (segment (start 101.051247 118.75) (end 100.801247 119) (width 0.25) (layer "F.Cu") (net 4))
 (segment (start 101.051247 113.75) (end 100.801247 114) (width 0.25) (layer "F.Cu") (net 4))
 (segment (start 155.55 121.15) (end 155.55 116.45) (width 0.25) (layer "B.Cu") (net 11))
 (segment (start 155.55 116.45) (end 157 115) (width 0.25) (layer "B.Cu") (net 11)))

